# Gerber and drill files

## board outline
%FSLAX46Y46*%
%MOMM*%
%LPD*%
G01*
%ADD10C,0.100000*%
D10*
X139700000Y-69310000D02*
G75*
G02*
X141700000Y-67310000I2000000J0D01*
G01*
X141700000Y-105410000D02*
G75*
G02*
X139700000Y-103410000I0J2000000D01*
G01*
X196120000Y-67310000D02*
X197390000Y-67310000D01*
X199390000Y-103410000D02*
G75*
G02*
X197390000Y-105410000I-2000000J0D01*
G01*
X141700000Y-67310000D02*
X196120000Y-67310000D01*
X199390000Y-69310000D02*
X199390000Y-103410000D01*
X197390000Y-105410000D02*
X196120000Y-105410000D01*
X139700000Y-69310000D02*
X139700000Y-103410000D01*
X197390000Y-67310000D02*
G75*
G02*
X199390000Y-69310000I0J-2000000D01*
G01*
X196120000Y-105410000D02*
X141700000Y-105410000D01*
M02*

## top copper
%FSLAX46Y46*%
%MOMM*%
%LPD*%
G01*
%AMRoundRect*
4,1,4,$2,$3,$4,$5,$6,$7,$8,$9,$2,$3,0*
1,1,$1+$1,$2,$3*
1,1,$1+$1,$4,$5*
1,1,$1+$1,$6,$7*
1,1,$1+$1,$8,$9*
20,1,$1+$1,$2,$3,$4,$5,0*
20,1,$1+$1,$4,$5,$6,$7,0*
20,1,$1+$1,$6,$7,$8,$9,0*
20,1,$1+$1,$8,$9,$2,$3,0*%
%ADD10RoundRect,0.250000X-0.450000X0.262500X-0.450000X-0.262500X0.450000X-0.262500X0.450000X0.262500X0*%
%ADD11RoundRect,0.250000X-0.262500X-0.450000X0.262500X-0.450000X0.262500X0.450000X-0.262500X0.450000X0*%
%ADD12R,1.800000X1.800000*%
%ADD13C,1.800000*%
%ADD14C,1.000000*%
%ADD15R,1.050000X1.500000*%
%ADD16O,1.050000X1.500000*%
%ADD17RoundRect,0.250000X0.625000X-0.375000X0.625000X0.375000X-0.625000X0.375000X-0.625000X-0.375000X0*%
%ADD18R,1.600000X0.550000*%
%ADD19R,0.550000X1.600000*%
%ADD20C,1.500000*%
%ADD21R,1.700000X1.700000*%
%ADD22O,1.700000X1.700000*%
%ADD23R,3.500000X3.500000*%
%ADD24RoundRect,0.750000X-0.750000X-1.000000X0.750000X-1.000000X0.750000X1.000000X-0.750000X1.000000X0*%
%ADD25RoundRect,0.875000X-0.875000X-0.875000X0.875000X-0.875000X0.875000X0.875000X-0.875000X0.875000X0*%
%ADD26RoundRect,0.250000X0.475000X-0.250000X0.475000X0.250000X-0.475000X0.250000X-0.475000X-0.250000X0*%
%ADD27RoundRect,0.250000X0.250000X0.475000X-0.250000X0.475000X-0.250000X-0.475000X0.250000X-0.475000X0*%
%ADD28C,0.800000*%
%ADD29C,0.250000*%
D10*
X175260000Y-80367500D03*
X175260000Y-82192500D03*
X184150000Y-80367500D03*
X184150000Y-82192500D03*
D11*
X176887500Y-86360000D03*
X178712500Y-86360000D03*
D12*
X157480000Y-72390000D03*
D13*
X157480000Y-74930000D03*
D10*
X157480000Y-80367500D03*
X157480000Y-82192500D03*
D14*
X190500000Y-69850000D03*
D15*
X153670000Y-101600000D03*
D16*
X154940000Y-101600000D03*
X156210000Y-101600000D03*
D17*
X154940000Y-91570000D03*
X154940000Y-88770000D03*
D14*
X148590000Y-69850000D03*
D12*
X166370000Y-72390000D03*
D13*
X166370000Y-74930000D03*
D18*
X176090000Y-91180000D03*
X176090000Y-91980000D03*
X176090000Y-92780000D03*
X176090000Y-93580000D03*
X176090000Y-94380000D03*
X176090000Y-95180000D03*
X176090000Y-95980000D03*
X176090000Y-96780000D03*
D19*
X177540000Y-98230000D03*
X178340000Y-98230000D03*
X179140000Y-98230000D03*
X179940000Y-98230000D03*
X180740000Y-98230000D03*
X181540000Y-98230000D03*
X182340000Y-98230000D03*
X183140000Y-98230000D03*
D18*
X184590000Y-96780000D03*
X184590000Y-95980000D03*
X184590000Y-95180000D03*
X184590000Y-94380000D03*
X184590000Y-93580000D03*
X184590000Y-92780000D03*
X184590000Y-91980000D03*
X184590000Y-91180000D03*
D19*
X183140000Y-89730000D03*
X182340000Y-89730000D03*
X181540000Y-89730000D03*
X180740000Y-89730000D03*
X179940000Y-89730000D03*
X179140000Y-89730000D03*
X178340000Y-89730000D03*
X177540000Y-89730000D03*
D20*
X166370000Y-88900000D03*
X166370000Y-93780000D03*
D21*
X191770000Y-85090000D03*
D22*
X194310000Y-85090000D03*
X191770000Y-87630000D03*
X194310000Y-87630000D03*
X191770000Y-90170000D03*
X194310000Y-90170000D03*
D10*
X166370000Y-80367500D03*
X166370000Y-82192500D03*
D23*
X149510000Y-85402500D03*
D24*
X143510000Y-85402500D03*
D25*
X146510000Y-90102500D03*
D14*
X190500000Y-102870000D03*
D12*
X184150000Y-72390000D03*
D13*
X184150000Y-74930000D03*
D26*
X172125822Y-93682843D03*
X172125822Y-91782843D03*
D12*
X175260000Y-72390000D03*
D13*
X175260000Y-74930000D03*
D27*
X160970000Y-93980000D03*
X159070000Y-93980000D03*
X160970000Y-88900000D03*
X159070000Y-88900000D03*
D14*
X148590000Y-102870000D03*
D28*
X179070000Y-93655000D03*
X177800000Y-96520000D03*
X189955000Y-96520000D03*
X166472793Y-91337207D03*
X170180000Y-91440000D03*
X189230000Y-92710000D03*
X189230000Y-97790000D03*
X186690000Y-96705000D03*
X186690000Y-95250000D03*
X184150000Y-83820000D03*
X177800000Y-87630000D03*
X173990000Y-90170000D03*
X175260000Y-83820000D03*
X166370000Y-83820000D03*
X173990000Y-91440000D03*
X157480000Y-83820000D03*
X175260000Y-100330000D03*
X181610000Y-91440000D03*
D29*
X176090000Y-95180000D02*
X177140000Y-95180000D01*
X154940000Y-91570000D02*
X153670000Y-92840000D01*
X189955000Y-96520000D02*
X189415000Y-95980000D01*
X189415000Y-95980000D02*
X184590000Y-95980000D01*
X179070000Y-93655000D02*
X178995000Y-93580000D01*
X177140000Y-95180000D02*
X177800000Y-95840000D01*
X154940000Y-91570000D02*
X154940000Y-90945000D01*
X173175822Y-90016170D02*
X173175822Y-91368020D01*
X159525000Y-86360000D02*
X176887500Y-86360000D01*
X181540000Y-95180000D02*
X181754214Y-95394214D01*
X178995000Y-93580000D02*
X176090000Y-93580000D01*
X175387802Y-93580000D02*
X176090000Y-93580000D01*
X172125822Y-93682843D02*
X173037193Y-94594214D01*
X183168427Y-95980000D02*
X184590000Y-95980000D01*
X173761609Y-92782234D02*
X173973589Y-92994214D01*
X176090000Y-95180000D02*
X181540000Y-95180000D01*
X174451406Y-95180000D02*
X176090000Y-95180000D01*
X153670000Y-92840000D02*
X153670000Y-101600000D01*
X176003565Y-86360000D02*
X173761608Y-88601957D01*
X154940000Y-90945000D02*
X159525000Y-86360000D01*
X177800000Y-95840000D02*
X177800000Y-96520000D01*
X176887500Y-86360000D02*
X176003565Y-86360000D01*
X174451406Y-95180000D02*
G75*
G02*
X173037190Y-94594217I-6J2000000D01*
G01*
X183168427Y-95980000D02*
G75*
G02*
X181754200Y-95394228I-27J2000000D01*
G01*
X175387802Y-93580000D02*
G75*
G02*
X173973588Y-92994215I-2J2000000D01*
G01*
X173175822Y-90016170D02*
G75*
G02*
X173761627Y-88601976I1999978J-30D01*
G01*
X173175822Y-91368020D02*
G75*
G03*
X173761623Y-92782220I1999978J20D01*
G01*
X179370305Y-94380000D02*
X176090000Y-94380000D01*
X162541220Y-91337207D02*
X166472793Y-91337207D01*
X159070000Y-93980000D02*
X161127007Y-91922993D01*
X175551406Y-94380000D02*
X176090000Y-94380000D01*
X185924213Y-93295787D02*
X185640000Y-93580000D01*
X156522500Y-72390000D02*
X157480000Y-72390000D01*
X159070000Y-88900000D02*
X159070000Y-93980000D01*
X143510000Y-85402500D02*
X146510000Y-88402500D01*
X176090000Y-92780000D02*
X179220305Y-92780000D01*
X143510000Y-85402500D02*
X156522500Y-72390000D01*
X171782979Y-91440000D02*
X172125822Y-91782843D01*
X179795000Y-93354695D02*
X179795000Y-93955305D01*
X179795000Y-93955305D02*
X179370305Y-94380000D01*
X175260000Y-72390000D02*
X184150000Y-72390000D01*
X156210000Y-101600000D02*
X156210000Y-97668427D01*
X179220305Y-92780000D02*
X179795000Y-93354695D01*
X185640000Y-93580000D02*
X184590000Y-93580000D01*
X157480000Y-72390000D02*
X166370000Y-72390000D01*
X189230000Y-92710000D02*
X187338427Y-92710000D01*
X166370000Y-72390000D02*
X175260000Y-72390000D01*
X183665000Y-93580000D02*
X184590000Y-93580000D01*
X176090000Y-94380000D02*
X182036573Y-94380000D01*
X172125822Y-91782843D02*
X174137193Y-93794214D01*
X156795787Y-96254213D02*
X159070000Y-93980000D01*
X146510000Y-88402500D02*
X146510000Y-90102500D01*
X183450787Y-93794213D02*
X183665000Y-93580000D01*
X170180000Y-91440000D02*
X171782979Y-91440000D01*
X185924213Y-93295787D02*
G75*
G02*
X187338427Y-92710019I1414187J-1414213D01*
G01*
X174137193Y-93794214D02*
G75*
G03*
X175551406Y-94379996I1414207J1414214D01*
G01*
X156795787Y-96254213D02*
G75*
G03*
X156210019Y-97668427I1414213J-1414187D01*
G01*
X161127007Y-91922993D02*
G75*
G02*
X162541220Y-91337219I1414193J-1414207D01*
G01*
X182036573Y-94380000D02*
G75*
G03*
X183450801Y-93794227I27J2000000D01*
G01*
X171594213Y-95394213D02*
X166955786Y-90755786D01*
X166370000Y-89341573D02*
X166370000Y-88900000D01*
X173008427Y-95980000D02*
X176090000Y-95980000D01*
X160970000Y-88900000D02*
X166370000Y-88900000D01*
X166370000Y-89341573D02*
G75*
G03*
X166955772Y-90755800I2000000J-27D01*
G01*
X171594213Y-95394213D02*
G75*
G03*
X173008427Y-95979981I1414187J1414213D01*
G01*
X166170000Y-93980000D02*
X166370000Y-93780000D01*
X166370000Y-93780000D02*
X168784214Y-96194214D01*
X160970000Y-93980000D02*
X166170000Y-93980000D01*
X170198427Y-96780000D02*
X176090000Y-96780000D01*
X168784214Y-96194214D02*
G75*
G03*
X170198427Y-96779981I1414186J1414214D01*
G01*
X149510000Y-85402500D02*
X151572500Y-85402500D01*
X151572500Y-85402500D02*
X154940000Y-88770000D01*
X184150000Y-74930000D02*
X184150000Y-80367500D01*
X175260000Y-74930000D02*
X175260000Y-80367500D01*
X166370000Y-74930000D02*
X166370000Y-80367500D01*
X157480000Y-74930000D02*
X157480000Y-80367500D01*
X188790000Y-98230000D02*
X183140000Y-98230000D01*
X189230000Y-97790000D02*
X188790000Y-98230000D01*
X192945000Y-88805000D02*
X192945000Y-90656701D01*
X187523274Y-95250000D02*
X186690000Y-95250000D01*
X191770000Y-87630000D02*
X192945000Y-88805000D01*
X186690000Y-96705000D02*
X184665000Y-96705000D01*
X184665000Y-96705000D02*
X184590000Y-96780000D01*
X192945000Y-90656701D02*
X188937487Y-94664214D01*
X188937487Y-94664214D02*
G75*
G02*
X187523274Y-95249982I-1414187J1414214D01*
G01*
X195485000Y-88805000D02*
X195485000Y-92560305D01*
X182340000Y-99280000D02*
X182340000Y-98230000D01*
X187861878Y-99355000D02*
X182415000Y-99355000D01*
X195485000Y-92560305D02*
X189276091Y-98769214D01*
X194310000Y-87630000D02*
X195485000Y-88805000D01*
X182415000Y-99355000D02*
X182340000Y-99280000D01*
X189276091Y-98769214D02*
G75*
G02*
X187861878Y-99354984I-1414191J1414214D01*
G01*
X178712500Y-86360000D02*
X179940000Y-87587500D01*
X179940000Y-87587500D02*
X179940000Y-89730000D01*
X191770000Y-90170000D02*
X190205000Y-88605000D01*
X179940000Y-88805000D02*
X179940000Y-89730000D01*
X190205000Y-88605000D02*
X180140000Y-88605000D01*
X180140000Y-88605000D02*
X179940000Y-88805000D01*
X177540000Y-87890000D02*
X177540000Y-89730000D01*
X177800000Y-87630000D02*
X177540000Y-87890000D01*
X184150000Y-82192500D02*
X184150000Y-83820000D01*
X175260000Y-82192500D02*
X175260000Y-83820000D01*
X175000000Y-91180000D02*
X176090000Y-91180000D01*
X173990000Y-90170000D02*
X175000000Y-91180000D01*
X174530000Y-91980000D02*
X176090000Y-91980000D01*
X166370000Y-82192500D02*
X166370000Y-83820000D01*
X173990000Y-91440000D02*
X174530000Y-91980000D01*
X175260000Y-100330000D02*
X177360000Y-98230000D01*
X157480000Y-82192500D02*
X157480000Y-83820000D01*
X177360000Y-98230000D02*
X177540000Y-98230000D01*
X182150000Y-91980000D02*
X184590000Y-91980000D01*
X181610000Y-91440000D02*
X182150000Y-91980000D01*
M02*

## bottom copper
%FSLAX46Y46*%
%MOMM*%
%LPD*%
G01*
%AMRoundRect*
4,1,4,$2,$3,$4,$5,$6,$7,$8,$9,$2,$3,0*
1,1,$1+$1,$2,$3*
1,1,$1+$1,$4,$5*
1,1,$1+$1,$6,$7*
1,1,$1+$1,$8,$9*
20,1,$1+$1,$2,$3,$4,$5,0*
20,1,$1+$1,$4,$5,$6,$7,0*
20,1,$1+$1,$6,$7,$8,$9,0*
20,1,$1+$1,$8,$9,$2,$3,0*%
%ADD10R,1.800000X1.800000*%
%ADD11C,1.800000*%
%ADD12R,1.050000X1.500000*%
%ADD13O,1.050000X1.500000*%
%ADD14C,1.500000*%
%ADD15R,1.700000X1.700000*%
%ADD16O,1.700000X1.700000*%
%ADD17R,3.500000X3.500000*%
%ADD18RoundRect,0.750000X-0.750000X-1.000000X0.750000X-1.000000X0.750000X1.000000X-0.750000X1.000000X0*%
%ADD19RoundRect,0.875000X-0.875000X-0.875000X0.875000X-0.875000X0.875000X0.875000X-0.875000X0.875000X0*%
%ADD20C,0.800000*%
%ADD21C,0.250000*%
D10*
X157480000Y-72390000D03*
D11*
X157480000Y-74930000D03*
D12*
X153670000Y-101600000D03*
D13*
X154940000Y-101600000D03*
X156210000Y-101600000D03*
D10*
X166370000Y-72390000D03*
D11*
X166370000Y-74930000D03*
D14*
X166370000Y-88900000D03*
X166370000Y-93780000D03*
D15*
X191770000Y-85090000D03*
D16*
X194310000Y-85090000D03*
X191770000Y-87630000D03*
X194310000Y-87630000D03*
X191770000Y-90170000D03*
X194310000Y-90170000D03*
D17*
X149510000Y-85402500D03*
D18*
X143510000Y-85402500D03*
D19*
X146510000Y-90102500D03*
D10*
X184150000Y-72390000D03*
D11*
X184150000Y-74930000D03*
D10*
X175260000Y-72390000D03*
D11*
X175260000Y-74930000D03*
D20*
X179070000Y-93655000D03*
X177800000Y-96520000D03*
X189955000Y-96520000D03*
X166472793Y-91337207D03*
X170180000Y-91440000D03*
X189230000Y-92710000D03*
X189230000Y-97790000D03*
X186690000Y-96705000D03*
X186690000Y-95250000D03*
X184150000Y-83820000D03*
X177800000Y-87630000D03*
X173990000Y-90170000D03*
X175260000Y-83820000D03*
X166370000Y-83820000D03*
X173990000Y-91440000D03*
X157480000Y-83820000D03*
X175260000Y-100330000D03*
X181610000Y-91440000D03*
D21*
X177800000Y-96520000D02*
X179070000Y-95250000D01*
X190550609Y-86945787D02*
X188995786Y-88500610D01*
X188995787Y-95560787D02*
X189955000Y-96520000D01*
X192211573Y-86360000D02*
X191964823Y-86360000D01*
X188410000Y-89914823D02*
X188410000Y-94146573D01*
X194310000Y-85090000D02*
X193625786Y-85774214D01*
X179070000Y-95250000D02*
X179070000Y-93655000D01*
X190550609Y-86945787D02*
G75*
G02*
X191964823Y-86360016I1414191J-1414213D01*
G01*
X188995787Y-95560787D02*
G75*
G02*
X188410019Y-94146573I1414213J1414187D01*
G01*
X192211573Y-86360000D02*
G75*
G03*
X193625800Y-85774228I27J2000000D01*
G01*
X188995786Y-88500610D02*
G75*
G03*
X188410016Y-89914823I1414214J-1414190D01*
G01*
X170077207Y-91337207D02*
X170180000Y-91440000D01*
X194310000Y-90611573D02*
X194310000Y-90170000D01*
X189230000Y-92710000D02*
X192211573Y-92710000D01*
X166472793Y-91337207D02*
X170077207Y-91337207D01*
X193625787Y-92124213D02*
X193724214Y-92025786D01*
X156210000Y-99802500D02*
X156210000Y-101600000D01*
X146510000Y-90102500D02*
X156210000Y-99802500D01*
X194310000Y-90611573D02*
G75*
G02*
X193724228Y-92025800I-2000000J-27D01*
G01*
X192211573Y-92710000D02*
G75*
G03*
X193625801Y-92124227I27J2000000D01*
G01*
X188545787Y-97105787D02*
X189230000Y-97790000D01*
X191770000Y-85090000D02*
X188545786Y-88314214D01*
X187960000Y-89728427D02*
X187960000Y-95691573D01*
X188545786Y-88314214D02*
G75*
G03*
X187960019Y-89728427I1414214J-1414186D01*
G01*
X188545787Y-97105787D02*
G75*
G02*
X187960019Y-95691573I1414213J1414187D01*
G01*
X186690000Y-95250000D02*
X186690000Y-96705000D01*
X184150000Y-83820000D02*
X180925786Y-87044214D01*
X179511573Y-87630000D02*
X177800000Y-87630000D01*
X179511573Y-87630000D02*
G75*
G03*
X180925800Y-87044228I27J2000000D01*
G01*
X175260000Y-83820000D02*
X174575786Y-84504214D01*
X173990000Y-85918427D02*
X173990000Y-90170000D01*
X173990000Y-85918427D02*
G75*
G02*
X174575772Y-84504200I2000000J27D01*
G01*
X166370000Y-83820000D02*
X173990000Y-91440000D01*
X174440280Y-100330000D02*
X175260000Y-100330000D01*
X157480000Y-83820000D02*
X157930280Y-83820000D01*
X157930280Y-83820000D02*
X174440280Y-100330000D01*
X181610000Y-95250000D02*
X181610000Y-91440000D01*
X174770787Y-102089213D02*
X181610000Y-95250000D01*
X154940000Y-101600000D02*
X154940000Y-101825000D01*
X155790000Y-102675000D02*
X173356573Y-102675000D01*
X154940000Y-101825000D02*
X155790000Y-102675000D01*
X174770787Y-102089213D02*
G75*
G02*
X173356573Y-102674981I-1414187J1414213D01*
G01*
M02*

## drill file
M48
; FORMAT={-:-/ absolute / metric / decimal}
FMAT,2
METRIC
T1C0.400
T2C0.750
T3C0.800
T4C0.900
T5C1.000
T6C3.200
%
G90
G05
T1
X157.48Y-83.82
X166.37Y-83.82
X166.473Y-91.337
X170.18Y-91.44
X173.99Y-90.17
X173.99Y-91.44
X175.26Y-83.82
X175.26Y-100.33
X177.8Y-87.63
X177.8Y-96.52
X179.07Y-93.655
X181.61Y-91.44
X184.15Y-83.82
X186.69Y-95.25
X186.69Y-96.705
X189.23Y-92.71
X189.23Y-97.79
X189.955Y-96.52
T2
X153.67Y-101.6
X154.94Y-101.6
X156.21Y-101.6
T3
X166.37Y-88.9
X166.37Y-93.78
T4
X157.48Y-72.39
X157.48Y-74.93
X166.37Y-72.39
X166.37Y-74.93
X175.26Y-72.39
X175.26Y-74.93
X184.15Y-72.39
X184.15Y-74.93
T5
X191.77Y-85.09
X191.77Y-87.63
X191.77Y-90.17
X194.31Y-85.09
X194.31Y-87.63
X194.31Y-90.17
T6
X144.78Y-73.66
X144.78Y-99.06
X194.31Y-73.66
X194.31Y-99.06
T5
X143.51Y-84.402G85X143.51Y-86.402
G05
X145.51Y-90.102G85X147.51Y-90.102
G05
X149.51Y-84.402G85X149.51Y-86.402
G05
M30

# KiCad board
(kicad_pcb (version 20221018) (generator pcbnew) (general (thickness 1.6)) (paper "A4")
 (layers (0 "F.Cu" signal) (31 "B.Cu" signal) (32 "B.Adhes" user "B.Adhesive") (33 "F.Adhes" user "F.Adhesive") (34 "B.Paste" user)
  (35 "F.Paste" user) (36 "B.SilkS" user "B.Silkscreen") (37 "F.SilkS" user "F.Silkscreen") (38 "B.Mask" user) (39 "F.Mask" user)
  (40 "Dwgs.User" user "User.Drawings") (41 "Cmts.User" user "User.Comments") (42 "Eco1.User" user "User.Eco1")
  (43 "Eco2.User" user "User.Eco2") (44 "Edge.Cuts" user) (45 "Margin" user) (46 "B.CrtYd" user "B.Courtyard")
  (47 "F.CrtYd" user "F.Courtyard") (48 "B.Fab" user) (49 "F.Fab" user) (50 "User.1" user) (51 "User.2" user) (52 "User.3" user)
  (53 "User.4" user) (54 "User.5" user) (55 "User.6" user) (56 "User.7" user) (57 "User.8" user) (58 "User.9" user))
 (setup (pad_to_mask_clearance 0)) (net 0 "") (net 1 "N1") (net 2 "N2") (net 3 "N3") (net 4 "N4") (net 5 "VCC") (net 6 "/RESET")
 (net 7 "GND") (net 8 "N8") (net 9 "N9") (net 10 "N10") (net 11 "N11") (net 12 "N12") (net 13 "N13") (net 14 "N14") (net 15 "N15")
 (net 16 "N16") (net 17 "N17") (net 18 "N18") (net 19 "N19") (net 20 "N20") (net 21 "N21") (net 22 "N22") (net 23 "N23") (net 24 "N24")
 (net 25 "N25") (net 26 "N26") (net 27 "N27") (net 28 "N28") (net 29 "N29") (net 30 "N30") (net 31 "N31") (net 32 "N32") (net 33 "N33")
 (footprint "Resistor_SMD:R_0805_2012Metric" (layer "F.Cu") (at 175.26 81.28 -90)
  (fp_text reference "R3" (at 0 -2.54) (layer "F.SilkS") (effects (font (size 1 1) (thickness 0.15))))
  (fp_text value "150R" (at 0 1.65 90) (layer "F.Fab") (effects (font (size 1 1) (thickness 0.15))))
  (pad "1" smd roundrect (at -0.9125 0 270) (size 1.025 1.4) (layers "F.Cu" "F.Paste" "F.Mask") (roundrect_rratio 0.243902439) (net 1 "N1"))
  (pad "2" smd roundrect (at 0.9125 0 270) (size 1.025 1.4) (layers "F.Cu" "F.Paste" "F.Mask") (roundrect_rratio 0.243902439) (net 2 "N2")))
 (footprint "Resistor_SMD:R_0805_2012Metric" (layer "F.Cu") (at 184.15 81.28 -90)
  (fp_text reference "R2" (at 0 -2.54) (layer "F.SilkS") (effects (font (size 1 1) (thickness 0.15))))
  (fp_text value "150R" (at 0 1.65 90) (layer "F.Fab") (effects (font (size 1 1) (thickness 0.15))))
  (pad "1" smd roundrect (at -0.9125 0 270) (size 1.025 1.4) (layers "F.Cu" "F.Paste" "F.Mask") (roundrect_rratio 0.243902439) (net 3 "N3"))
  (pad "2" smd roundrect (at 0.9125 0 270) (size 1.025 1.4) (layers "F.Cu" "F.Paste" "F.Mask") (roundrect_rratio 0.243902439) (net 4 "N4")))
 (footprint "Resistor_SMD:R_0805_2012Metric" (layer "F.Cu") (at 177.8 86.36)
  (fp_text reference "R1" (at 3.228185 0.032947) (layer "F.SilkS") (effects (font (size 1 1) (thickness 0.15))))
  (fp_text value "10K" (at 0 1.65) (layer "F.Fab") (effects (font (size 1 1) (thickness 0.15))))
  (pad "1" smd roundrect (at -0.9125 0) (size 1.025 1.4) (layers "F.Cu" "F.Paste" "F.Mask") (roundrect_rratio 0.243902439) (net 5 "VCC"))
  (pad "2" smd roundrect (at 0.9125 0) (size 1.025 1.4) (layers "F.Cu" "F.Paste" "F.Mask") (roundrect_rratio 0.243902439) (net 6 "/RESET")))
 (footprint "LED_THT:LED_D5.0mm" (layer "F.Cu") (at 157.48 72.39 -90)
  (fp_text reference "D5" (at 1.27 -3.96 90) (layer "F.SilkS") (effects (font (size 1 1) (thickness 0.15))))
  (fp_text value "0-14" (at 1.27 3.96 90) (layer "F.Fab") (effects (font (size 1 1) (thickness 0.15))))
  (pad "1" thru_hole rect (at 0 0 270) (size 1.8 1.8) (drill 0.9) (layers "*.Cu" "*.Mask") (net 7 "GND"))
  (pad "2" thru_hole circle (at 2.54 0 270) (size 1.8 1.8) (drill 0.9) (layers "*.Cu" "*.Mask") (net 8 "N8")))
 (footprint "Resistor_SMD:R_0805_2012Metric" (layer "F.Cu") (at 157.48 81.28 -90)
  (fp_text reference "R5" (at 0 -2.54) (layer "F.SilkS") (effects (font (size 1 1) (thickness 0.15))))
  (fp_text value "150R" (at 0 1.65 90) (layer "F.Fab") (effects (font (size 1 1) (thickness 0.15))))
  (pad "1" smd roundrect (at -0.9125 0 270) (size 1.025 1.4) (layers "F.Cu" "F.Paste" "F.Mask") (roundrect_rratio 0.243902439) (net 8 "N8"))
  (pad "2" smd roundrect (at 0.9125 0 270) (size 1.025 1.4) (layers "F.Cu" "F.Paste" "F.Mask") (roundrect_rratio 0.243902439) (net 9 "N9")))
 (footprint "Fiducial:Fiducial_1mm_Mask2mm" (layer "F.Cu") (at 190.5 69.85)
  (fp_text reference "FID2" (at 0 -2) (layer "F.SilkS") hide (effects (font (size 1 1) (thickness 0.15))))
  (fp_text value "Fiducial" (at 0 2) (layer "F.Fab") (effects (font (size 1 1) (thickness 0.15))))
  (pad "" smd circle (at 0 0) (size 1 1) (layers "F.Cu" "F.Mask") (solder_mask_margin 0.5) (clearance 0.5)))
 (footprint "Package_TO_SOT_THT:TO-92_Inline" (layer "F.Cu") (at 153.67 101.6)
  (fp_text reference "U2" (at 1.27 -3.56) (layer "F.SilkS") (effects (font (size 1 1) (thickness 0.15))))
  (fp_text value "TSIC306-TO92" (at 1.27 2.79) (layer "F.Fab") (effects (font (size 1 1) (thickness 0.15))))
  (pad "1" thru_hole rect (at 0 0) (size 1.05 1.5) (drill 0.75) (layers "*.Cu" "*.Mask") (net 5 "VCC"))
  (pad "2" thru_hole oval (at 1.27 0) (size 1.05 1.5) (drill 0.75) (layers "*.Cu" "*.Mask") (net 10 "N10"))
  (pad "3" thru_hole oval (at 2.54 0) (size 1.05 1.5) (drill 0.75) (layers "*.Cu" "*.Mask") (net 7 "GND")))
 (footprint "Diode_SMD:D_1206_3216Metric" (layer "F.Cu") (at 154.94 90.17 90)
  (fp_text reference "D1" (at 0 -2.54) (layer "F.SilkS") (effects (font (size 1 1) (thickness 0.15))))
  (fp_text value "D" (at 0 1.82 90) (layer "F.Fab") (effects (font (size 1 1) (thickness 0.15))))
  (pad "1" smd roundrect (at -1.4 0 90) (size 1.25 1.75) (layers "F.Cu" "F.Paste" "F.Mask") (roundrect_rratio 0.2) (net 5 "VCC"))
  (pad "2" smd roundrect (at 1.4 0 90) (size 1.25 1.75) (layers "F.Cu" "F.Paste" "F.Mask") (roundrect_rratio 0.2) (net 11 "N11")))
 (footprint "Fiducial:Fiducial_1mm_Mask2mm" (layer "F.Cu") (at 148.59 69.85)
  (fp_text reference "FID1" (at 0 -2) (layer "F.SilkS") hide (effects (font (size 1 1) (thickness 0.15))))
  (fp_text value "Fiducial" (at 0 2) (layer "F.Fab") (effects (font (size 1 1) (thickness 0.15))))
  (pad "" smd circle (at 0 0) (size 1 1) (layers "F.Cu" "F.Mask") (solder_mask_margin 0.5) (clearance 0.5)))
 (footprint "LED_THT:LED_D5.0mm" (layer "F.Cu") (at 166.37 72.39 -90)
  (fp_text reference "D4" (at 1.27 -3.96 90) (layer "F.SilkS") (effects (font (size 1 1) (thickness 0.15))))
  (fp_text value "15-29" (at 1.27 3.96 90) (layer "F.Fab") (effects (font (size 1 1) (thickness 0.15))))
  (pad "1" thru_hole rect (at 0 0 270) (size 1.8 1.8) (drill 0.9) (layers "*.Cu" "*.Mask") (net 7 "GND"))
  (pad "2" thru_hole circle (at 2.54 0 270) (size 1.8 1.8) (drill 0.9) (layers "*.Cu" "*.Mask") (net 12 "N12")))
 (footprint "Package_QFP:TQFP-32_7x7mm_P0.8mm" (layer "F.Cu") (at 180.34 93.98)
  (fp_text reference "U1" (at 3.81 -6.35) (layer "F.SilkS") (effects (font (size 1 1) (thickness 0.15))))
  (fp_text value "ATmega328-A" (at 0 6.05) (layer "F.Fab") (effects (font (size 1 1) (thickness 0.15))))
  (pad "1" smd rect (at -4.25 -2.8) (size 1.6 0.55) (layers "F.Cu" "F.Paste" "F.Mask") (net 2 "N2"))
  (pad "2" smd rect (at -4.25 -2) (size 1.6 0.55) (layers "F.Cu" "F.Paste" "F.Mask") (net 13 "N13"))
  (pad "3" smd rect (at -4.25 -1.2) (size 1.6 0.55) (layers "F.Cu" "F.Paste" "F.Mask") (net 7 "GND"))
  (pad "4" smd rect (at -4.25 -0.4) (size 1.6 0.55) (layers "F.Cu" "F.Paste" "F.Mask") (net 5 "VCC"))
  (pad "5" smd rect (at -4.25 0.4) (size 1.6 0.55) (layers "F.Cu" "F.Paste" "F.Mask") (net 7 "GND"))
  (pad "6" smd rect (at -4.25 1.2) (size 1.6 0.55) (layers "F.Cu" "F.Paste" "F.Mask") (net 5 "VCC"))
  (pad "7" smd rect (at -4.25 2) (size 1.6 0.55) (layers "F.Cu" "F.Paste" "F.Mask") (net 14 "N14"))
  (pad "8" smd rect (at -4.25 2.8) (size 1.6 0.55) (layers "F.Cu" "F.Paste" "F.Mask") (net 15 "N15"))
  (pad "9" smd rect (at -2.8 4.25 90) (size 1.6 0.55) (layers "F.Cu" "F.Paste" "F.Mask") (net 9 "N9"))
  (pad "10" smd rect (at -2 4.25 90) (size 1.6 0.55) (layers "F.Cu" "F.Paste" "F.Mask") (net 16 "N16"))
  (pad "11" smd rect (at -1.2 4.25 90) (size 1.6 0.55) (layers "F.Cu" "F.Paste" "F.Mask") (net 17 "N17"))
  (pad "12" smd rect (at -0.4 4.25 90) (size 1.6 0.55) (layers "F.Cu" "F.Paste" "F.Mask") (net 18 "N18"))
  (pad "13" smd rect (at 0.4 4.25 90) (size 1.6 0.55) (layers "F.Cu" "F.Paste" "F.Mask") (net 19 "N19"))
  (pad "14" smd rect (at 1.2 4.25 90) (size 1.6 0.55) (layers "F.Cu" "F.Paste" "F.Mask") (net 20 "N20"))
  (pad "15" smd rect (at 2 4.25 90) (size 1.6 0.55) (layers "F.Cu" "F.Paste" "F.Mask") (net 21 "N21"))
  (pad "16" smd rect (at 2.8 4.25 90) (size 1.6 0.55) (layers "F.Cu" "F.Paste" "F.Mask") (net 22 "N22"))
  (pad "17" smd rect (at 4.25 2.8) (size 1.6 0.55) (layers "F.Cu" "F.Paste" "F.Mask") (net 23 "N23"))
  (pad "18" smd rect (at 4.25 2) (size 1.6 0.55) (layers "F.Cu" "F.Paste" "F.Mask") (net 5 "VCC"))
  (pad "19" smd rect (at 4.25 1.2) (size 1.6 0.55) (layers "F.Cu" "F.Paste" "F.Mask") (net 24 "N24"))
  (pad "20" smd rect (at 4.25 0.4) (size 1.6 0.55) (layers "F.Cu" "F.Paste" "F.Mask") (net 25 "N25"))
  (pad "21" smd rect (at 4.25 -0.4) (size 1.6 0.55) (layers "F.Cu" "F.Paste" "F.Mask") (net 7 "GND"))
  (pad "22" smd rect (at 4.25 -1.2) (size 1.6 0.55) (layers "F.Cu" "F.Paste" "F.Mask") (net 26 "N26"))
  (pad "23" smd rect (at 4.25 -2) (size 1.6 0.55) (layers "F.Cu" "F.Paste" "F.Mask") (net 10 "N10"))
  (pad "24" smd rect (at 4.25 -2.8) (size 1.6 0.55) (layers "F.Cu" "F.Paste" "F.Mask") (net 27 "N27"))
  (pad "25" smd rect (at 2.8 -4.25 90) (size 1.6 0.55) (layers "F.Cu" "F.Paste" "F.Mask") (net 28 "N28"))
  (pad "26" smd rect (at 2 -4.25 90) (size 1.6 0.55) (layers "F.Cu" "F.Paste" "F.Mask") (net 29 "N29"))
  (pad "27" smd rect (at 1.2 -4.25 90) (size 1.6 0.55) (layers "F.Cu" "F.Paste" "F.Mask") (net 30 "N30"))
  (pad "28" smd rect (at 0.4 -4.25 90) (size 1.6 0.55) (layers "F.Cu" "F.Paste" "F.Mask") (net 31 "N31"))
  (pad "29" smd rect (at -0.4 -4.25 90) (size 1.6 0.55) (layers "F.Cu" "F.Paste" "F.Mask") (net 6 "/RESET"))
  (pad "30" smd rect (at -1.2 -4.25 90) (size 1.6 0.55) (layers "F.Cu" "F.Paste" "F.Mask") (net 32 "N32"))
  (pad "31" smd rect (at -2 -4.25 90) (size 1.6 0.55) (layers "F.Cu" "F.Paste" "F.Mask") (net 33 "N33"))
  (pad "32" smd rect (at -2.8 -4.25 90) (size 1.6 0.55) (layers "F.Cu" "F.Paste" "F.Mask") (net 4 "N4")))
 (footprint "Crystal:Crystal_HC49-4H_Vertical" (layer "F.Cu") (at 166.37 88.9 -90)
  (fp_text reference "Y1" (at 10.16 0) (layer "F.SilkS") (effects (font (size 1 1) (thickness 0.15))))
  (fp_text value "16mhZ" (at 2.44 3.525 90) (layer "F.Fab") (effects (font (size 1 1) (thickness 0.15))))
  (pad "1" thru_hole circle (at 0 0 270) (size 1.5 1.5) (drill 0.8) (layers "*.Cu" "*.Mask") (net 14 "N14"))
  (pad "2" thru_hole circle (at 4.88 0 270) (size 1.5 1.5) (drill 0.8) (layers "*.Cu" "*.Mask") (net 15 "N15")))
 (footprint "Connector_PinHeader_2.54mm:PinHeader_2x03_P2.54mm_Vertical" (layer "F.Cu") (at 191.77 85.09)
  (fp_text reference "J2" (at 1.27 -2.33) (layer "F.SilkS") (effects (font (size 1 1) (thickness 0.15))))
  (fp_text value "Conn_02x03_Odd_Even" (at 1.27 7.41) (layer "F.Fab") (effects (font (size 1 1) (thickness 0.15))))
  (pad "1" thru_hole rect (at 0 0) (size 1.7 1.7) (drill 1) (layers "*.Cu" "*.Mask") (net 22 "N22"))
  (pad "2" thru_hole oval (at 2.54 0) (size 1.7 1.7) (drill 1) (layers "*.Cu" "*.Mask") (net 5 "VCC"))
  (pad "3" thru_hole oval (at 0 2.54) (size 1.7 1.7) (drill 1) (layers "*.Cu" "*.Mask") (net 23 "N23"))
  (pad "4" thru_hole oval (at 2.54 2.54) (size 1.7 1.7) (drill 1) (layers "*.Cu" "*.Mask") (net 21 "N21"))
  (pad "5" thru_hole oval (at 0 5.08) (size 1.7 1.7) (drill 1) (layers "*.Cu" "*.Mask") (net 6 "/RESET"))
  (pad "6" thru_hole oval (at 2.54 5.08) (size 1.7 1.7) (drill 1) (layers "*.Cu" "*.Mask") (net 7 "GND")))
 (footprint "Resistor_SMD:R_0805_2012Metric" (layer "F.Cu") (at 166.37 81.28 -90)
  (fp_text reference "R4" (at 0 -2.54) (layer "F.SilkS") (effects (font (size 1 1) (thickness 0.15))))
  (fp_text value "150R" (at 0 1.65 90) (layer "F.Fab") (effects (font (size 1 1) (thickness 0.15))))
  (pad "1" smd roundrect (at -0.9125 0 270) (size 1.025 1.4) (layers "F.Cu" "F.Paste" "F.Mask") (roundrect_rratio 0.243902439)
   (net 12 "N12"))
  (pad "2" smd roundrect (at 0.9125 0 270) (size 1.025 1.4) (layers "F.Cu" "F.Paste" "F.Mask") (roundrect_rratio 0.243902439) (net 13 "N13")))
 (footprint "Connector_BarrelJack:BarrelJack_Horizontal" (layer "F.Cu") (at 149.51 85.4025)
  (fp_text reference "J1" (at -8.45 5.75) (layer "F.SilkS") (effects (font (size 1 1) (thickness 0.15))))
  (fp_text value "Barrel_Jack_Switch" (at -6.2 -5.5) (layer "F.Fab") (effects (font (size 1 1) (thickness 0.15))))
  (pad "1" thru_hole rect (at 0 0) (size 3.5 3.5) (drill oval 1 3) (layers "*.Cu" "*.Mask") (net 11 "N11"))
  (pad "2" thru_hole roundrect (at -6 0) (size 3 3.5) (drill oval 1 3) (layers "*.Cu" "*.Mask") (roundrect_rratio 0.25) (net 7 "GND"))
  (pad "3" thru_hole roundrect (at -3 4.7) (size 3.5 3.5) (drill oval 3 1) (layers "*.Cu" "*.Mask") (roundrect_rratio 0.25) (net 7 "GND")))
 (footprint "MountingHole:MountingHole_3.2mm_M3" (layer "F.Cu") (at 144.78 99.06)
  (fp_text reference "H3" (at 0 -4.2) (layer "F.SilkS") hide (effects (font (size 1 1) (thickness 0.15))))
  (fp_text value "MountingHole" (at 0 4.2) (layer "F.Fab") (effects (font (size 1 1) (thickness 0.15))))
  (pad "" np_thru_hole circle (at 0 0) (size 3.2 3.2) (drill 3.2) (layers "*.Cu" "*.Mask")))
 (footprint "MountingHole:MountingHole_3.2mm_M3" (layer "F.Cu") (at 194.31 73.66)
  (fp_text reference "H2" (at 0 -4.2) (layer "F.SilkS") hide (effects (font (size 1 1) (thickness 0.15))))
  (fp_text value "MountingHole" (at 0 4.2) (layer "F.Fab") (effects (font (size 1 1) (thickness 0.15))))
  (pad "" np_thru_hole circle (at 0 0) (size 3.2 3.2) (drill 3.2) (layers "*.Cu" "*.Mask")))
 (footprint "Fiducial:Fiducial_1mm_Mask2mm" (layer "F.Cu") (at 190.5 102.87)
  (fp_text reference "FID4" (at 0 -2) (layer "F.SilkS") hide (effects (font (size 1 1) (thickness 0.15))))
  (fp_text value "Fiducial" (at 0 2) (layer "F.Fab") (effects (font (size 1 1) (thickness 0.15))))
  (pad "" smd circle (at 0 0) (size 1 1) (layers "F.Cu" "F.Mask") (solder_mask_margin 0.5) (clearance 0.5)))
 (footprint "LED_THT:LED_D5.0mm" (layer "F.Cu") (at 184.15 72.39 -90)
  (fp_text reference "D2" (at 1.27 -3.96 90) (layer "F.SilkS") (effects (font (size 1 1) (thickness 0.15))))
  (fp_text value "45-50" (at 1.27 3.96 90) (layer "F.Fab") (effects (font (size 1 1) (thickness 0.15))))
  (pad "1" thru_hole rect (at 0 0 270) (size 1.8 1.8) (drill 0.9) (layers "*.Cu" "*.Mask") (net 7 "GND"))
  (pad "2" thru_hole circle (at 2.54 0 270) (size 1.8 1.8) (drill 0.9) (layers "*.Cu" "*.Mask") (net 3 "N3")))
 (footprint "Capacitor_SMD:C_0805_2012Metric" (layer "F.Cu") (at 172.125822 92.732843 90)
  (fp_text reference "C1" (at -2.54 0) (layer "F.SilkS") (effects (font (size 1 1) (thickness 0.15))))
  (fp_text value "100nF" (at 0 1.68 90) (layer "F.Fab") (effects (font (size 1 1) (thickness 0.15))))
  (pad "1" smd roundrect (at -0.95 0 90) (size 1 1.45) (layers "F.Cu" "F.Paste" "F.Mask") (roundrect_rratio 0.25) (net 5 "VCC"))
  (pad "2" smd roundrect (at 0.95 0 90) (size 1 1.45) (layers "F.Cu" "F.Paste" "F.Mask") (roundrect_rratio 0.25) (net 7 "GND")))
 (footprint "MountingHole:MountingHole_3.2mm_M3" (layer "F.Cu") (at 144.78 73.66)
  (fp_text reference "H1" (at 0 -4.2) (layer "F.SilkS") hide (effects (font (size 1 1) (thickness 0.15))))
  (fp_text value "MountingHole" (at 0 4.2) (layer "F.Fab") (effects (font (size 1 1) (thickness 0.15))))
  (pad "" np_thru_hole circle (at 0 0) (size 3.2 3.2) (drill 3.2) (layers "*.Cu" "*.Mask")))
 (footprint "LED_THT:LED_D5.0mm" (layer "F.Cu") (at 175.26 72.39 -90)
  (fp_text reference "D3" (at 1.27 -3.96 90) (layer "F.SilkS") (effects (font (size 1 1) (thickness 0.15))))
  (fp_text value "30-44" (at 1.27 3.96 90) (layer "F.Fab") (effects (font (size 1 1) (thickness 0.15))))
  (pad "1" thru_hole rect (at 0 0 270) (size 1.8 1.8) (drill 0.9) (layers "*.Cu" "*.Mask") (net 7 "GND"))
  (pad "2" thru_hole circle (at 2.54 0 270) (size 1.8 1.8) (drill 0.9) (layers "*.Cu" "*.Mask") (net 1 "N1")))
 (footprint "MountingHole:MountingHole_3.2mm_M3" (layer "F.Cu") (at 194.31 99.06)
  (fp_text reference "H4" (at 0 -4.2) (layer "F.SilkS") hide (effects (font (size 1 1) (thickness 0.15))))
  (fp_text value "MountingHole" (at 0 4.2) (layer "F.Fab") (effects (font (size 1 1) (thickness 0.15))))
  (pad "" np_thru_hole circle (at 0 0) (size 3.2 3.2) (drill 3.2) (layers "*.Cu" "*.Mask")))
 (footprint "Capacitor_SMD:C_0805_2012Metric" (layer "F.Cu") (at 160.02 93.98 180)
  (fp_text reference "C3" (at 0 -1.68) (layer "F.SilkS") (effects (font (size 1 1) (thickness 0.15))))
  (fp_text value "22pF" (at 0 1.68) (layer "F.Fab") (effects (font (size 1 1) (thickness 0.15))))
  (pad "1" smd roundrect (at -0.95 0 180) (size 1 1.45) (layers "F.Cu" "F.Paste" "F.Mask") (roundrect_rratio 0.25) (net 15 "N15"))
  (pad "2" smd roundrect (at 0.95 0 180) (size 1 1.45) (layers "F.Cu" "F.Paste" "F.Mask") (roundrect_rratio 0.25) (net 7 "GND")))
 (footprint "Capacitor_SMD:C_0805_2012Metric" (layer "F.Cu") (at 160.02 88.9 180)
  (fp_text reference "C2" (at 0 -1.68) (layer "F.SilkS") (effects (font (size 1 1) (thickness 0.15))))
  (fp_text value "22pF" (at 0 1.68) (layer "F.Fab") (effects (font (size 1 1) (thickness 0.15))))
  (pad "1" smd roundrect (at -0.95 0 180) (size 1 1.45) (layers "F.Cu" "F.Paste" "F.Mask") (roundrect_rratio 0.25) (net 14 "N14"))
  (pad "2" smd roundrect (at 0.95 0 180) (size 1 1.45) (layers "F.Cu" "F.Paste" "F.Mask") (roundrect_rratio 0.25) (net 7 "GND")))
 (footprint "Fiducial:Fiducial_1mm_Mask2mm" (layer "F.Cu") (at 148.59 102.87)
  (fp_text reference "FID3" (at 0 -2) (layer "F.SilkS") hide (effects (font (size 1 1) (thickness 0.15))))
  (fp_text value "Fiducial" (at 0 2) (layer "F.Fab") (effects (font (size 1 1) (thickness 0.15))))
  (pad "" smd circle (at 0 0) (size 1 1) (layers "F.Cu" "F.Mask") (solder_mask_margin 0.5) (clearance 0.5)))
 (gr_arc (start 139.7 69.31) (mid 140.285786 67.895786) (end 141.7 67.31) (stroke (width 0.1) (type default)) (layer "Edge.Cuts"))
 (gr_arc (start 141.7 105.41) (mid 140.285786 104.824214) (end 139.7 103.41) (stroke (width 0.1) (type default)) (layer "Edge.Cuts"))
 (gr_line (start 196.12 67.31) (end 197.39 67.31) (stroke (width 0.1) (type default)) (layer "Edge.Cuts"))
 (gr_arc (start 199.39 103.41) (mid 198.804214 104.824214) (end 197.39 105.41) (stroke (width 0.1) (type default)) (layer "Edge.Cuts"))
 (gr_line (start 141.7 67.31) (end 196.12 67.31) (stroke (width 0.1) (type default)) (layer "Edge.Cuts"))
 (gr_line (start 199.39 69.31) (end 199.39 103.41) (stroke (width 0.1) (type default)) (layer "Edge.Cuts"))
 (gr_line (start 197.39 105.41) (end 196.12 105.41) (stroke (width 0.1) (type default)) (layer "Edge.Cuts"))
 (gr_line (start 139.7 69.31) (end 139.7 103.41) (stroke (width 0.1) (type default)) (layer "Edge.Cuts"))
 (gr_arc (start 197.39 67.31) (mid 198.804214 67.895786) (end 199.39 69.31) (stroke (width 0.1) (type default)) (layer "Edge.Cuts"))
 (gr_line (start 196.12 105.41) (end 141.7 105.41) (stroke (width 0.1) (type default)) (layer "Edge.Cuts"))
 (segment (start 176.09 95.18) (end 177.14 95.18) (width 0.25) (layer "F.Cu") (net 5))
 (segment (start 154.94 91.57) (end 153.67 92.84) (width 0.25) (layer "F.Cu") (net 5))
 (segment (start 189.955 96.52) (end 189.415 95.98) (width 0.25) (layer "F.Cu") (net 5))
 (segment (start 189.415 95.98) (end 184.59 95.98) (width 0.25) (layer "F.Cu") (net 5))
 (segment (start 179.07 93.655) (end 178.995 93.58) (width 0.25) (layer "F.Cu") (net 5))
 (segment (start 177.14 95.18) (end 177.8 95.84) (width 0.25) (layer "F.Cu") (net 5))
 (segment (start 154.94 91.57) (end 154.94 90.945) (width 0.25) (layer "F.Cu") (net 5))
 (segment (start 173.175822 90.01617) (end 173.175822 91.36802) (width 0.25) (layer "F.Cu") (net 5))
 (segment (start 159.525 86.36) (end 176.8875 86.36) (width 0.25) (layer "F.Cu") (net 5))
 (segment (start 181.54 95.18) (end 181.754214 95.394214) (width 0.25) (layer "F.Cu") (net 5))
 (segment (start 178.995 93.58) (end 176.09 93.58) (width 0.25) (layer "F.Cu") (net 5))
 (segment (start 175.387802 93.58) (end 176.09 93.58) (width 0.25) (layer "F.Cu") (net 5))
 (segment (start 172.125822 93.682843) (end 173.037193 94.594214) (width 0.25) (layer "F.Cu") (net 5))
 (segment (start 183.168427 95.98) (end 184.59 95.98) (width 0.25) (layer "F.Cu") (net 5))
 (segment (start 173.761609 92.782234) (end 173.973589 92.994214) (width 0.25) (layer "F.Cu") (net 5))
 (segment (start 176.09 95.18) (end 181.54 95.18) (width 0.25) (layer "F.Cu") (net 5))
 (segment (start 174.451406 95.18) (end 176.09 95.18) (width 0.25) (layer "F.Cu") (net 5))
 (segment (start 153.67 92.84) (end 153.67 101.6) (width 0.25) (layer "F.Cu") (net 5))
 (segment (start 176.003565 86.36) (end 173.761608 88.601957) (width 0.25) (layer "F.Cu") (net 5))
 (segment (start 154.94 90.945) (end 159.525 86.36) (width 0.25) (layer "F.Cu") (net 5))
 (segment (start 177.8 95.84) (end 177.8 96.52) (width 0.25) (layer "F.Cu") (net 5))
 (segment (start 176.8875 86.36) (end 176.003565 86.36) (width 0.25) (layer "F.Cu") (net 5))
 (via (at 179.07 93.655) (size 0.8) (drill 0.4) (layers "F.Cu" "B.Cu") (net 5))
 (via (at 177.8 96.52) (size 0.8) (drill 0.4) (layers "F.Cu" "B.Cu") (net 5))
 (via (at 189.955 96.52) (size 0.8) (drill 0.4) (layers "F.Cu" "B.Cu") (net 5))
 (arc (start 174.451406 95.18) (mid 173.686039 95.027759) (end 173.037193 94.594214) (width 0.25) (layer "F.Cu") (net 5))
 (arc (start 183.168427 95.98) (mid 182.40306 95.827759) (end 181.754214 95.394214) (width 0.25) (layer "F.Cu") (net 5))
 (arc (start 175.387802 93.58) (mid 174.622435 93.427759) (end 173.973589 92.994214) (width 0.25) (layer "F.Cu") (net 5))
 (arc (start 173.175822 90.01617) (mid 173.328063 89.250803) (end 173.761608 88.601957) (width 0.25) (layer "F.Cu") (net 5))
 (arc (start 173.175822 91.36802) (mid 173.328063 92.133387) (end 173.761609 92.782234) (width 0.25) (layer "F.Cu") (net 5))
 (segment (start 177.8 96.52) (end 179.07 95.25) (width 0.25) (layer "B.Cu") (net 5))
 (segment (start 190.550609 86.945787) (end 188.995786 88.50061) (width 0.25) (layer "B.Cu") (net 5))
 (segment (start 188.995787 95.560787) (end 189.955 96.52) (width 0.25) (layer "B.Cu") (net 5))
 (segment (start 192.211573 86.36) (end 191.964823 86.36) (width 0.25) (layer "B.Cu") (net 5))
 (segment (start 188.41 89.914823) (end 188.41 94.146573) (width 0.25) (layer "B.Cu") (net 5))
 (segment (start 194.31 85.09) (end 193.625786 85.774214) (width 0.25) (layer "B.Cu") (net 5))
 (segment (start 179.07 95.25) (end 179.07 93.655) (width 0.25) (layer "B.Cu") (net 5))
 (arc (start 190.550609 86.945787) (mid 191.199456 86.512241) (end 191.964823 86.36) (width 0.25) (layer "B.Cu") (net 5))
 (arc (start 188.995787 95.560787) (mid 188.562241 94.91194) (end 188.41 94.146573) (width 0.25) (layer "B.Cu") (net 5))
 (arc (start 192.211573 86.36) (mid 192.97694 86.207759) (end 193.625786 85.774214) (width 0.25) (layer "B.Cu") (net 5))
 (arc (start 188.995786 88.50061) (mid 188.562241 89.149456) (end 188.41 89.914823) (width 0.25) (layer "B.Cu") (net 5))
 (segment (start 179.370305 94.38) (end 176.09 94.38) (width 0.25) (layer "F.Cu") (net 7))
 (segment (start 162.54122 91.337207) (end 166.472793 91.337207) (width 0.25) (layer "F.Cu") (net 7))
 (segment (start 159.07 93.98) (end 161.127007 91.922993) (width 0.25) (layer "F.Cu") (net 7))
 (segment (start 175.551406 94.38) (end 176.09 94.38) (width 0.25) (layer "F.Cu") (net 7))
 (segment (start 185.924213 93.295787) (end 185.64 93.58) (width 0.25) (layer "F.Cu") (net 7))
 (segment (start 156.5225 72.39) (end 157.48 72.39) (width 0.25) (layer "F.Cu") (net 7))
 (segment (start 159.07 88.9) (end 159.07 93.98) (width 0.25) (layer "F.Cu") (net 7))
 (segment (start 143.51 85.4025) (end 146.51 88.4025) (width 0.25) (layer "F.Cu") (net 7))
 (segment (start 176.09 92.78) (end 179.220305 92.78) (width 0.25) (layer "F.Cu") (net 7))
 (segment (start 143.51 85.4025) (end 156.5225 72.39) (width 0.25) (layer "F.Cu") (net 7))
 (segment (start 171.782979 91.44) (end 172.125822 91.782843) (width 0.25) (layer "F.Cu") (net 7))
 (segment (start 179.795 93.354695) (end 179.795 93.955305) (width 0.25) (layer "F.Cu") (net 7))
 (segment (start 179.795 93.955305) (end 179.370305 94.38) (width 0.25) (layer "F.Cu") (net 7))
 (segment (start 175.26 72.39) (end 184.15 72.39) (width 0.25) (layer "F.Cu") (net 7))
 (segment (start 156.21 101.6) (end 156.21 97.668427) (width 0.25) (layer "F.Cu") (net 7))
 (segment (start 179.220305 92.78) (end 179.795 93.354695) (width 0.25) (layer "F.Cu") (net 7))
 (segment (start 185.64 93.58) (end 184.59 93.58) (width 0.25) (layer "F.Cu") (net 7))
 (segment (start 157.48 72.39) (end 166.37 72.39) (width 0.25) (layer "F.Cu") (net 7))
 (segment (start 189.23 92.71) (end 187.338427 92.71) (width 0.25) (layer "F.Cu") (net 7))
 (segment (start 166.37 72.39) (end 175.26 72.39) (width 0.25) (layer "F.Cu") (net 7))
 (segment (start 183.665 93.58) (end 184.59 93.58) (width 0.25) (layer "F.Cu") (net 7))
 (segment (start 176.09 94.38) (end 182.036573 94.38) (width 0.25) (layer "F.Cu") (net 7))
 (segment (start 172.125822 91.782843) (end 174.137193 93.794214) (width 0.25) (layer "F.Cu") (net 7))
 (segment (start 156.795787 96.254213) (end 159.07 93.98) (width 0.25) (layer "F.Cu") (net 7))
 (segment (start 146.51 88.4025) (end 146.51 90.1025) (width 0.25) (layer "F.Cu") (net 7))
 (segment (start 183.450787 93.794213) (end 183.665 93.58) (width 0.25) (layer "F.Cu") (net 7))
 (segment (start 170.18 91.44) (end 171.782979 91.44) (width 0.25) (layer "F.Cu") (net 7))
 (via (at 166.472793 91.337207) (size 0.8) (drill 0.4) (layers "F.Cu" "B.Cu") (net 7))
 (via (at 170.18 91.44) (size 0.8) (drill 0.4) (layers "F.Cu" "B.Cu") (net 7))
 (via (at 189.23 92.71) (size 0.8) (drill 0.4) (layers "F.Cu" "B.Cu") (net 7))
 (arc (start 185.924213 93.295787) (mid 186.57306 92.862241) (end 187.338427 92.71) (width 0.25) (layer "F.Cu") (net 7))
 (arc (start 174.137193 93.794214) (mid 174.786039 94.227759) (end 175.551406 94.38) (width 0.25) (layer "F.Cu") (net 7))
 (arc (start 156.795787 96.254213) (mid 156.362241 96.90306) (end 156.21 97.668427) (width 0.25) (layer "F.Cu") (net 7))
 (arc (start 161.127007 91.922993) (mid 161.775853 91.489448) (end 162.54122 91.337207) (width 0.25) (layer "F.Cu") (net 7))
 (arc (start 182.036573 94.38) (mid 182.80194 94.227759) (end 183.450787 93.794213) (width 0.25) (layer "F.Cu") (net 7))
 (segment (start 170.077207 91.337207) (end 170.18 91.44) (width 0.25) (layer "B.Cu") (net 7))
 (segment (start 194.31 90.611573) (end 194.31 90.17) (width 0.25) (layer "B.Cu") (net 7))
 (segment (start 189.23 92.71) (end 192.211573 92.71) (width 0.25) (layer "B.Cu") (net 7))
 (segment (start 166.472793 91.337207) (end 170.077207 91.337207) (width 0.25) (layer "B.Cu") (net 7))
 (segment (start 193.625787 92.124213) (end 193.724214 92.025786) (width 0.25) (layer "B.Cu") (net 7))
 (segment (start 156.21 99.8025) (end 156.21 101.6) (width 0.25) (layer "B.Cu") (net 7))
 (segment (start 146.51 90.1025) (end 156.21 99.8025) (width 0.25) (layer "B.Cu") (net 7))
 (arc (start 194.31 90.611573) (mid 194.157759 91.37694) (end 193.724214 92.025786) (width 0.25) (layer "B.Cu") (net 7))
 (arc (start 192.211573 92.71) (mid 192.97694 92.557759) (end 193.625787 92.124213) (width 0.25) (layer "B.Cu") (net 7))
 (segment (start 171.594213 95.394213) (end 166.955786 90.755786) (width 0.25) (layer "F.Cu") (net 14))
 (segment (start 166.37 89.341573) (end 166.37 88.9) (width 0.25) (layer "F.Cu") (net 14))
 (segment (start 173.008427 95.98) (end 176.09 95.98) (width 0.25) (layer "F.Cu") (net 14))
 (segment (start 160.97 88.9) (end 166.37 88.9) (width 0.25) (layer "F.Cu") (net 14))
 (arc (start 166.37 89.341573) (mid 166.522241 90.10694) (end 166.955786 90.755786) (width 0.25) (layer "F.Cu") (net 14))
 (arc (start 171.594213 95.394213) (mid 172.24306 95.827759) (end 173.008427 95.98) (width 0.25) (layer "F.Cu") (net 14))
 (segment (start 166.17 93.98) (end 166.37 93.78) (width 0.25) (layer "F.Cu") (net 15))
 (segment (start 166.37 93.78) (end 168.784214 96.194214) (width 0.25) (layer "F.Cu") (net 15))
 (segment (start 160.97 93.98) (end 166.17 93.98) (width 0.25) (layer "F.Cu") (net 15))
 (segment (start 170.198427 96.78) (end 176.09 96.78) (width 0.25) (layer "F.Cu") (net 15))
 (arc (start 168.784214 96.194214) (mid 169.43306 96.627759) (end 170.198427 96.78) (width 0.25) (layer "F.Cu") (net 15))
 (segment (start 149.51 85.4025) (end 151.5725 85.4025) (width 0.25) (layer "F.Cu") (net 11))
 (segment (start 151.5725 85.4025) (end 154.94 88.77) (width 0.25) (layer "F.Cu") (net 11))
 (segment (start 184.15 74.93) (end 184.15 80.3675) (width 0.25) (layer "F.Cu") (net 3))
 (segment (start 175.26 74.93) (end 175.26 80.3675) (width 0.25) (layer "F.Cu") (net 1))
 (segment (start 166.37 74.93) (end 166.37 80.3675) (width 0.25) (layer "F.Cu") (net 12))
 (segment (start 157.48 74.93) (end 157.48 80.3675) (width 0.25) (layer "F.Cu") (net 8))
 (segment (start 188.79 98.23) (end 183.14 98.23) (width 0.25) (layer "F.Cu") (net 22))
 (segment (start 189.23 97.79) (end 188.79 98.23) (width 0.25) (layer "F.Cu") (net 22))
 (via (at 189.23 97.79) (size 0.8) (drill 0.4) (layers "F.Cu" "B.Cu") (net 22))
 (segment (start 188.545787 97.105787) (end 189.23 97.79) (width 0.25) (layer "B.Cu") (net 22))
 (segment (start 191.77 85.09) (end 188.545786 88.314214) (width 0.25) (layer "B.Cu") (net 22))
 (segment (start 187.96 89.728427) (end 187.96 95.691573) (width 0.25) (layer "B.Cu") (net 22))
 (arc (start 188.545786 88.314214) (mid 188.112241 88.96306) (end 187.96 89.728427) (width 0.25) (layer "B.Cu") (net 22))
 (arc (start 188.545787 97.105787) (mid 188.112241 96.45694) (end 187.96 95.691573) (width 0.25) (layer "B.Cu") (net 22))
 (segment (start 192.945 88.805) (end 192.945 90.656701) (width 0.25) (layer "F.Cu") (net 23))
 (segment (start 187.523274 95.25) (end 186.69 95.25) (width 0.25) (layer "F.Cu") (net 23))
 (segment (start 191.77 87.63) (end 192.945 88.805) (width 0.25) (layer "F.Cu") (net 23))
 (segment (start 186.69 96.705) (end 184.665 96.705) (width 0.25) (layer "F.Cu") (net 23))
 (segment (start 184.665 96.705) (end 184.59 96.78) (width 0.25) (layer "F.Cu") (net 23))
 (segment (start 192.945 90.656701) (end 188.937487 94.664214) (width 0.25) (layer "F.Cu") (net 23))
 (via (at 186.69 96.705) (size 0.8) (drill 0.4) (layers "F.Cu" "B.Cu") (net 23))
 (via (at 186.69 95.25) (size 0.8) (drill 0.4) (layers "F.Cu" "B.Cu") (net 23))
 (arc (start 188.937487 94.664214) (mid 188.288641 95.097759) (end 187.523274 95.25) (width 0.25) (layer "F.Cu") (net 23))
 (segment (start 186.69 95.25) (end 186.69 96.705) (width 0.25) (layer "B.Cu") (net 23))
 (segment (start 195.485 88.805) (end 195.485 92.560305) (width 0.25) (layer "F.Cu") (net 21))
 (segment (start 182.34 99.28) (end 182.34 98.23) (width 0.25) (layer "F.Cu") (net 21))
 (segment (start 187.861878 99.355) (end 182.415 99.355) (width 0.25) (layer "F.Cu") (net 21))
 (segment (start 195.485 92.560305) (end 189.276091 98.769214) (width 0.25) (layer "F.Cu") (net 21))
 (segment (start 194.31 87.63) (end 195.485 88.805) (width 0.25) (layer "F.Cu") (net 21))
 (segment (start 182.415 99.355) (end 182.34 99.28) (width 0.25) (layer "F.Cu") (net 21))
 (arc (start 189.276091 98.769214) (mid 188.627245 99.202759) (end 187.861878 99.355) (width 0.25) (layer "F.Cu") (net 21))
 (segment (start 178.7125 86.36) (end 179.94 87.5875) (width 0.25) (layer "F.Cu") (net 6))
 (segment (start 179.94 87.5875) (end 179.94 89.73) (width 0.25) (layer "F.Cu") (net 6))
 (segment (start 191.77 90.17) (end 190.205 88.605) (width 0.25) (layer "F.Cu") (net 6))
 (segment (start 179.94 88.805) (end 179.94 89.73) (width 0.25) (layer "F.Cu") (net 6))
 (segment (start 190.205 88.605) (end 180.14 88.605) (width 0.25) (layer "F.Cu") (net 6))
 (segment (start 180.14 88.605) (end 179.94 88.805) (width 0.25) (layer "F.Cu") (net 6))
 (segment (start 177.54 87.89) (end 177.54 89.73) (width 0.25) (layer "F.Cu") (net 4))
 (segment (start 177.8 87.63) (end 177.54 87.89) (width 0.25) (layer "F.Cu") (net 4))
 (segment (start 184.15 82.1925) (end 184.15 83.82) (width 0.25) (layer "F.Cu") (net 4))
 (via (at 184.15 83.82) (size 0.8) (drill 0.4) (layers "F.Cu" "B.Cu") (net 4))
 (via (at 177.8 87.63) (size 0.8) (drill 0.4) (layers "F.Cu" "B.Cu") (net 4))
 (segment (start 184.15 83.82) (end 180.925786 87.044214) (width 0.25) (layer "B.Cu") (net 4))
 (segment (start 179.511573 87.63) (end 177.8 87.63) (width 0.25) (layer "B.Cu") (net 4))
 (arc (start 179.511573 87.63) (mid 180.27694 87.477759) (end 180.925786 87.044214) (width 0.25) (layer "B.Cu") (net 4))
 (segment (start 175.26 82.1925) (end 175.26 83.82) (width 0.25) (layer "F.Cu") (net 2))
 (segment (start 175 91.18) (end 176.09 91.18) (width 0.25) (layer "F.Cu") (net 2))
 (segment (start 173.99 90.17) (end 175 91.18) (width 0.25) (layer "F.Cu") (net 2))
 (via (at 173.99 90.17) (size 0.8) (drill 0.4) (layers "F.Cu" "B.Cu") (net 2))
 (via (at 175.26 83.82) (size 0.8) (drill 0.4) (layers "F.Cu" "B.Cu") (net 2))
 (segment (start 175.26 83.82) (end 174.575786 84.504214) (width 0.25) (layer "B.Cu") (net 2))
 (segment (start 173.99 85.918427) (end 173.99 90.17) (width 0.25) (layer "B.Cu") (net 2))
 (arc (start 173.99 85.918427) (mid 174.142241 85.15306) (end 174.575786 84.504214) (width 0.25) (layer "B.Cu") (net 2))
 (segment (start 174.53 91.98) (end 176.09 91.98) (width 0.25) (layer "F.Cu") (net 13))
 (segment (start 166.37 82.1925) (end 166.37 83.82) (width 0.25) (layer "F.Cu") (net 13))
 (segment (start 173.99 91.44) (end 174.53 91.98) (width 0.25) (layer "F.Cu") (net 13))
 (via (at 166.37 83.82) (size 0.8) (drill 0.4) (layers "F.Cu" "B.Cu") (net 13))
 (via (at 173.99 91.44) (size 0.8) (drill 0.4) (layers "F.Cu" "B.Cu") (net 13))
 (segment (start 166.37 83.82) (end 173.99 91.44) (width 0.25) (layer "B.Cu") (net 13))
 (segment (start 175.26 100.33) (end 177.36 98.23) (width 0.25) (layer "F.Cu") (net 9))
 (segment (start 157.48 82.1925) (end 157.48 83.82) (width 0.25) (layer "F.Cu") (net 9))
 (segment (start 177.36 98.23) (end 177.54 98.23) (width 0.25) (layer "F.Cu") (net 9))
 (via (at 157.48 83.82) (size 0.8) (drill 0.4) (layers "F.Cu" "B.Cu") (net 9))
 (via (at 175.26 100.33) (size 0.8) (drill 0.4) (layers "F.Cu" "B.Cu") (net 9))
 (segment (start 174.44028 100.33) (end 175.26 100.33) (width 0.25) (layer "B.Cu") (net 9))
 (segment (start 157.48 83.82) (end 157.93028 83.82) (width 0.25) (layer "B.Cu") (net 9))
 (segment (start 157.93028 83.82) (end 174.44028 100.33) (width 0.25) (layer "B.Cu") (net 9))
 (segment (start 182.15 91.98) (end 184.59 91.98) (width 0.25) (layer "F.Cu") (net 10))
 (segment (start 181.61 91.44) (end 182.15 91.98) (width 0.25) (layer "F.Cu") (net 10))
 (via (at 181.61 91.44) (size 0.8) (drill 0.4) (layers "F.Cu" "B.Cu") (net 10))
 (segment (start 181.61 95.25) (end 181.61 91.44) (width 0.25) (layer "B.Cu") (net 10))
 (segment (start 174.770787 102.089213) (end 181.61 95.25) (width 0.25) (layer "B.Cu") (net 10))
 (segment (start 154.94 101.6) (end 154.94 101.825) (width 0.25) (layer "B.Cu") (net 10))
 (segment (start 155.79 102.675) (end 173.356573 102.675) (width 0.25) (layer "B.Cu") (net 10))
 (segment (start 154.94 101.825) (end 155.79 102.675) (width 0.25) (layer "B.Cu") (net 10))
 (arc (start 174.770787 102.089213) (mid 174.12194 102.522759) (end 173.356573 102.675) (width 0.25) (layer "B.Cu") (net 10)))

